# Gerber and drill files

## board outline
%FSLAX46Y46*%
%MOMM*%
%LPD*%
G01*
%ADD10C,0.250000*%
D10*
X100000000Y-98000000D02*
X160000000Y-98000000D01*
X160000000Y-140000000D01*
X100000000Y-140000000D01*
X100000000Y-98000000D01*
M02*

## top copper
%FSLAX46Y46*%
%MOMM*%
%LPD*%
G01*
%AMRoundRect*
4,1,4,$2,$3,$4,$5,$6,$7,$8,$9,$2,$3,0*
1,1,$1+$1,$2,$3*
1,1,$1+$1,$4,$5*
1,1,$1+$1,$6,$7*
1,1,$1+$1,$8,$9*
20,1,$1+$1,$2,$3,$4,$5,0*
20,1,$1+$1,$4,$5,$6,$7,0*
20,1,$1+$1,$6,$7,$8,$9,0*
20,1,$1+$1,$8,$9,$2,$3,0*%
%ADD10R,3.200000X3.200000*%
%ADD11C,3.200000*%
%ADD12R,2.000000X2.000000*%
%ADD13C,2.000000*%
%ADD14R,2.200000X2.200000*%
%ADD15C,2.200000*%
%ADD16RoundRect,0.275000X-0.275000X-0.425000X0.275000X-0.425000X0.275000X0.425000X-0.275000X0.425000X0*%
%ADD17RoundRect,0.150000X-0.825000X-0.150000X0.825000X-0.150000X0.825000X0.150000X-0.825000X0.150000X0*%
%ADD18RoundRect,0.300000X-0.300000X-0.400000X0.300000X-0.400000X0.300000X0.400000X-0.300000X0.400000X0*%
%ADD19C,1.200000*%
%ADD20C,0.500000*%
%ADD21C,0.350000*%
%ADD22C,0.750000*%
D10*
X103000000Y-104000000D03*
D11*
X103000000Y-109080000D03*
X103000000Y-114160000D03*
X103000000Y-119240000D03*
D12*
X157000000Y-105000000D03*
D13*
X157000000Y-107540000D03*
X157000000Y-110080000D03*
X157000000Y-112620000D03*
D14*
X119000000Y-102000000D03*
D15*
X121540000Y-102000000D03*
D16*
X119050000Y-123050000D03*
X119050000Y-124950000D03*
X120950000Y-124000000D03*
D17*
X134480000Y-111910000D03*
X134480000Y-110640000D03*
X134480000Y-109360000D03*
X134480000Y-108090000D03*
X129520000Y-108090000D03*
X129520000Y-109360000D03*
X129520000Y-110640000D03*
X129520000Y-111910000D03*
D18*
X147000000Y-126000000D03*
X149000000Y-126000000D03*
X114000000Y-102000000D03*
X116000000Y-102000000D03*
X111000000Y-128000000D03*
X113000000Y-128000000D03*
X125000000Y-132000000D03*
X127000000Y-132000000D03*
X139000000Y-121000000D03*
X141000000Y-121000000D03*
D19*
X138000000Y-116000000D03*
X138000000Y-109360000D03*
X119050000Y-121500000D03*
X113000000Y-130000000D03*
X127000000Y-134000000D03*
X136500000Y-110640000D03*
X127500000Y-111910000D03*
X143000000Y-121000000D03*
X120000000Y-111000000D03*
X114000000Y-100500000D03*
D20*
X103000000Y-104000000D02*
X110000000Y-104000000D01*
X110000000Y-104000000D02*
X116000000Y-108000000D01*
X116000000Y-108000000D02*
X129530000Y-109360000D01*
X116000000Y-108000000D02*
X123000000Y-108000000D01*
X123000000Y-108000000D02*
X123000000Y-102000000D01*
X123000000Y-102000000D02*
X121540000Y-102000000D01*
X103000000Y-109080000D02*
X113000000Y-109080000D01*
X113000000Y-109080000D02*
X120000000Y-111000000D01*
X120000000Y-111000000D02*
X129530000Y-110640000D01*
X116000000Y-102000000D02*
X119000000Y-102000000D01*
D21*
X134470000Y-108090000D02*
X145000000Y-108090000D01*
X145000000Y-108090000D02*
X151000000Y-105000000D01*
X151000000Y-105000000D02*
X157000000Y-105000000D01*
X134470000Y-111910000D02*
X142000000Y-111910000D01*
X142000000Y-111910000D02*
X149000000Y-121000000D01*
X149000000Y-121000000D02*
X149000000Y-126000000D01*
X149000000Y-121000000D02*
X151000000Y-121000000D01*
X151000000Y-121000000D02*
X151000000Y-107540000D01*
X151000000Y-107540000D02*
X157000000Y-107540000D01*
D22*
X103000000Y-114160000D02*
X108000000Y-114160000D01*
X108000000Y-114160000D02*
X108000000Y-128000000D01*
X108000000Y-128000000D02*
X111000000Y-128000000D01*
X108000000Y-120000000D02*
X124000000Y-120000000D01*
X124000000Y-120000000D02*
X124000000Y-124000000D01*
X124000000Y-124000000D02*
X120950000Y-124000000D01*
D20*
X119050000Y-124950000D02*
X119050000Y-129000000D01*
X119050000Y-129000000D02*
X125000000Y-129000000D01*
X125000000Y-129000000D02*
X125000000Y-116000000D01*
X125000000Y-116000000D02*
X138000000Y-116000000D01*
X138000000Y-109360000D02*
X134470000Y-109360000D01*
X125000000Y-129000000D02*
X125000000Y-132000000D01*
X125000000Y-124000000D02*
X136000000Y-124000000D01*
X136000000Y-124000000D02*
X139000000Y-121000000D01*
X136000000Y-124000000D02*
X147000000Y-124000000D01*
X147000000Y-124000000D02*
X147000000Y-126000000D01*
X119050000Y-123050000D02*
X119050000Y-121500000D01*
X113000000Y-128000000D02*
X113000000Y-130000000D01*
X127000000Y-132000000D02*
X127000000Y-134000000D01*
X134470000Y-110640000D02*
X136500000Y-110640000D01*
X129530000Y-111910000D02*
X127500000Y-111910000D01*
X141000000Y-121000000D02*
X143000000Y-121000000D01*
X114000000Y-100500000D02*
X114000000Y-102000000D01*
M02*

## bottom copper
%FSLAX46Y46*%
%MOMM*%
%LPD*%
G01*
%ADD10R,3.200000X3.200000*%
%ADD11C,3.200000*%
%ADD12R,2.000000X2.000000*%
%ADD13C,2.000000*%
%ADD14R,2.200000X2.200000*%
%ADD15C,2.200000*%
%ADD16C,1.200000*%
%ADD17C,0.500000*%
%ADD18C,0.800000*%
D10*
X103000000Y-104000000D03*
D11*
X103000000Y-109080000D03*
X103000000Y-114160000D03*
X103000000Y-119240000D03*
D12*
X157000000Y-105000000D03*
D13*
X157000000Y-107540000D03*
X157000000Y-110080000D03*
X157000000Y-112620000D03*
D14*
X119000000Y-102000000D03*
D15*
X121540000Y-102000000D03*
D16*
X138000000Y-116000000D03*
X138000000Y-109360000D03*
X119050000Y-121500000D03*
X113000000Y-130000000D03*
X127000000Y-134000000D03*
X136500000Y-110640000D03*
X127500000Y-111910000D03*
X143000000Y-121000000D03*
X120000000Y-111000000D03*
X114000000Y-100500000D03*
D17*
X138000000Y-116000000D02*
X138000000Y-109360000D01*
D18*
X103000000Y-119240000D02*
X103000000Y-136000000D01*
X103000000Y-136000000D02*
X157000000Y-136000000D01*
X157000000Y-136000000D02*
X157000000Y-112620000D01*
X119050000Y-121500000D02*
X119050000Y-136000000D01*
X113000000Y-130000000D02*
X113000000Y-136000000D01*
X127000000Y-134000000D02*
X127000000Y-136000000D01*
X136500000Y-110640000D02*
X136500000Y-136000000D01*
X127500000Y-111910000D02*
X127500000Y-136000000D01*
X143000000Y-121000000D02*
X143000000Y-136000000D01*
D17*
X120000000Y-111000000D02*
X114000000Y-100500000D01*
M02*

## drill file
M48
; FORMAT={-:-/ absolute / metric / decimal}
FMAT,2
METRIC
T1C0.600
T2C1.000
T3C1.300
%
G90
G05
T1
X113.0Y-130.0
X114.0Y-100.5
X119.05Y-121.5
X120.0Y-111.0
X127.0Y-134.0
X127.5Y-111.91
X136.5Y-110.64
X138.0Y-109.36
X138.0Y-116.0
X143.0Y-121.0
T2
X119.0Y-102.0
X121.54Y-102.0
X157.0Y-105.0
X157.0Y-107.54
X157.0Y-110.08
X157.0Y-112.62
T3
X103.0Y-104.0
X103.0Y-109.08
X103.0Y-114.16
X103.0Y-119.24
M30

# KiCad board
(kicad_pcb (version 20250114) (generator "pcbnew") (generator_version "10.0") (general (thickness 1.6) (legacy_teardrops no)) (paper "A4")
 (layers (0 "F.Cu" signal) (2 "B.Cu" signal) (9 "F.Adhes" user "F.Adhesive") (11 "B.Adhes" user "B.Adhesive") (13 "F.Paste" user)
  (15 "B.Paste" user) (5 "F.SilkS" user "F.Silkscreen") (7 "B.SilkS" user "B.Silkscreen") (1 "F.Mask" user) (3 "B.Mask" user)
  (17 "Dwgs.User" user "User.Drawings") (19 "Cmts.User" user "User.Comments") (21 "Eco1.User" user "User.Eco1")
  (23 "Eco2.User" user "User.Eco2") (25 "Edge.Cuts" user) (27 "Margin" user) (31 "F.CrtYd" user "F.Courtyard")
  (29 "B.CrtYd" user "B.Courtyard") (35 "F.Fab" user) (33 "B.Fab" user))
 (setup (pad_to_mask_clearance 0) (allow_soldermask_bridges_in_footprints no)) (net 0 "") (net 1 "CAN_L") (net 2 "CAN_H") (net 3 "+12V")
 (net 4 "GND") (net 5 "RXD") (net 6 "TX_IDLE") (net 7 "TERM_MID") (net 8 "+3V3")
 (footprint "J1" (layer "F.Cu") (at 103.00 104.00 0)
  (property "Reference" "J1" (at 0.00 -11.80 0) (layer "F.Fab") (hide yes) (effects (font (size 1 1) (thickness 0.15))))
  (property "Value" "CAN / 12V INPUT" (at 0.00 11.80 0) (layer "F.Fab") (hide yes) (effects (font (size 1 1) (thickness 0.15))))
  (pad "1" thru_hole rect (at 0.00 0.00) (size 3.20 3.20) (drill 1.30) (layers "*.Cu" "*.Mask") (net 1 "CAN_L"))
  (pad "2" thru_hole circle (at 0.00 5.08) (size 3.20 3.20) (drill 1.30) (layers "*.Cu" "*.Mask") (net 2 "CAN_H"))
  (pad "3" thru_hole circle (at 0.00 10.16) (size 3.20 3.20) (drill 1.30) (layers "*.Cu" "*.Mask") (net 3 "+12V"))
  (pad "4" thru_hole circle (at 0.00 15.24) (size 3.20 3.20) (drill 1.30) (layers "*.Cu" "*.Mask") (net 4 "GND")))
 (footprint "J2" (layer "F.Cu") (at 157.00 105.00 0)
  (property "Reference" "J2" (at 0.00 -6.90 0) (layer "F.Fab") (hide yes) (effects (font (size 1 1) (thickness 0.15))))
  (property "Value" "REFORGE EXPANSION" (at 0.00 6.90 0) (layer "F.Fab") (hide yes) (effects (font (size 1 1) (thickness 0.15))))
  (pad "1" thru_hole rect (at 0.00 0.00) (size 2.00 2.00) (drill 1.00) (layers "*.Cu" "*.Mask") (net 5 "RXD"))
  (pad "2" thru_hole circle (at 0.00 2.54) (size 2.00 2.00) (drill 1.00) (layers "*.Cu" "*.Mask") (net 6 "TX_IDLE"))
  (pad "3" thru_hole circle (at 0.00 5.08) (size 2.00 2.00) (drill 1.00) (layers "*.Cu" "*.Mask") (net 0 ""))
  (pad "4" thru_hole circle (at 0.00 7.62) (size 2.00 2.00) (drill 1.00) (layers "*.Cu" "*.Mask") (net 4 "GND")))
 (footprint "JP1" (layer "F.Cu") (at 119.00 102.00 0)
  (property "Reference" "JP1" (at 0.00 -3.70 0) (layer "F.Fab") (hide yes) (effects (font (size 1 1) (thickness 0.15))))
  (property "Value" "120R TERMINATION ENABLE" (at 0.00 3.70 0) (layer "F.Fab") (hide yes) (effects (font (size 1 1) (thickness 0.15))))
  (pad "1" thru_hole rect (at 0.00 0.00) (size 2.20 2.20) (drill 1.00) (layers "*.Cu" "*.Mask") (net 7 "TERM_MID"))
  (pad "2" thru_hole circle (at 2.54 0.00) (size 2.20 2.20) (drill 1.00) (layers "*.Cu" "*.Mask") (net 1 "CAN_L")))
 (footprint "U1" (layer "F.Cu") (at 120.00 124.00 0)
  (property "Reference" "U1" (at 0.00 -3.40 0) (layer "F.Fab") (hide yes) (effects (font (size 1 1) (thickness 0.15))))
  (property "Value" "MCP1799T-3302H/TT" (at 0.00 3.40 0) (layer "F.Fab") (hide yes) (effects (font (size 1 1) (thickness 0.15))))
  (pad "1" smd roundrect (at -0.95 -0.95) (size 1.10 1.40) (layers "F.Cu" "F.Paste" "F.Mask") (roundrect_rratio 0.25) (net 4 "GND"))
  (pad "2" smd roundrect (at -0.95 0.95) (size 1.10 1.40) (layers "F.Cu" "F.Paste" "F.Mask") (roundrect_rratio 0.25) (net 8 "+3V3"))
  (pad "3" smd roundrect (at 0.95 0.00) (size 1.10 1.40) (layers "F.Cu" "F.Paste" "F.Mask") (roundrect_rratio 0.25) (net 3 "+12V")))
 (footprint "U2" (layer "F.Cu") (at 132.00 110.00 180)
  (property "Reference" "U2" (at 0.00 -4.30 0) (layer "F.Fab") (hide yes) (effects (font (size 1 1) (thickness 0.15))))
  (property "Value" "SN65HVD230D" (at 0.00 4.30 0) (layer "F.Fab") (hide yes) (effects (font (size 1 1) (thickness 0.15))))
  (pad "1" smd roundrect (at -2.48 -1.91) (size 1.95 0.60) (layers "F.Cu" "F.Paste" "F.Mask") (roundrect_rratio 0.25) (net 6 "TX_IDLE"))
  (pad "2" smd roundrect (at -2.48 -0.64) (size 1.95 0.60) (layers "F.Cu" "F.Paste" "F.Mask") (roundrect_rratio 0.25) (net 4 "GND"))
  (pad "3" smd roundrect (at -2.48 0.64) (size 1.95 0.60) (layers "F.Cu" "F.Paste" "F.Mask") (roundrect_rratio 0.25) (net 8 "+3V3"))
  (pad "4" smd roundrect (at -2.48 1.91) (size 1.95 0.60) (layers "F.Cu" "F.Paste" "F.Mask") (roundrect_rratio 0.25) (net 5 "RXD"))
  (pad "5" smd roundrect (at 2.48 1.91) (size 1.95 0.60) (layers "F.Cu" "F.Paste" "F.Mask") (roundrect_rratio 0.25) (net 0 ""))
  (pad "6" smd roundrect (at 2.48 0.64) (size 1.95 0.60) (layers "F.Cu" "F.Paste" "F.Mask") (roundrect_rratio 0.25) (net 1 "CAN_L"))
  (pad "7" smd roundrect (at 2.48 -0.64) (size 1.95 0.60) (layers "F.Cu" "F.Paste" "F.Mask") (roundrect_rratio 0.25) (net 2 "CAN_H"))
  (pad "8" smd roundrect (at 2.48 -1.91) (size 1.95 0.60) (layers "F.Cu" "F.Paste" "F.Mask") (roundrect_rratio 0.25) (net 4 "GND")))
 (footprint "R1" (layer "F.Cu") (at 148.00 126.00 0)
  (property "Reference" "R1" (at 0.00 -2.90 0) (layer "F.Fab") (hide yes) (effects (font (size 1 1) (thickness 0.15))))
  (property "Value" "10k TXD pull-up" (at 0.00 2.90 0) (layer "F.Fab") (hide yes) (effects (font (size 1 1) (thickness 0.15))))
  (pad "1" smd roundrect (at -1.00 0.00) (size 1.20 1.40) (layers "F.Cu" "F.Paste" "F.Mask") (roundrect_rratio 0.25) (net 8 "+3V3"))
  (pad "2" smd roundrect (at 1.00 0.00) (size 1.20 1.40) (layers "F.Cu" "F.Paste" "F.Mask") (roundrect_rratio 0.25) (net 6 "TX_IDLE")))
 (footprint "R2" (layer "F.Cu") (at 115.00 102.00 0)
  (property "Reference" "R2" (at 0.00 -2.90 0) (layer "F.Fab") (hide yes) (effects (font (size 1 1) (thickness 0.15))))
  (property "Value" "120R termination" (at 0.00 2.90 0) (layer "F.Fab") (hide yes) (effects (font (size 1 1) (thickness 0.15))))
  (pad "1" smd roundrect (at -1.00 0.00) (size 1.20 1.40) (layers "F.Cu" "F.Paste" "F.Mask") (roundrect_rratio 0.25) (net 2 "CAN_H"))
  (pad "2" smd roundrect (at 1.00 0.00) (size 1.20 1.40) (layers "F.Cu" "F.Paste" "F.Mask") (roundrect_rratio 0.25) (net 7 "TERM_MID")))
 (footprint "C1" (layer "F.Cu") (at 112.00 128.00 0)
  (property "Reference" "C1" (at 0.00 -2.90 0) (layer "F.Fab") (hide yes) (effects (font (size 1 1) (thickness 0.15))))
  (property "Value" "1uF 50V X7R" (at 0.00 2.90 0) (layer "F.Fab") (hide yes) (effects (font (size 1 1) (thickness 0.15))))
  (pad "1" smd roundrect (at -1.00 0.00) (size 1.20 1.40) (layers "F.Cu" "F.Paste" "F.Mask") (roundrect_rratio 0.25) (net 3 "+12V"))
  (pad "2" smd roundrect (at 1.00 0.00) (size 1.20 1.40) (layers "F.Cu" "F.Paste" "F.Mask") (roundrect_rratio 0.25) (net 4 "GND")))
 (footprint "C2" (layer "F.Cu") (at 126.00 132.00 0)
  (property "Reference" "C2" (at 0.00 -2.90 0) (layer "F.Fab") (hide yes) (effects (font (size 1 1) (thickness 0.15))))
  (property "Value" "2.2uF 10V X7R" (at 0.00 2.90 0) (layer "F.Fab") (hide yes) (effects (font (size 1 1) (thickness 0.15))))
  (pad "1" smd roundrect (at -1.00 0.00) (size 1.20 1.40) (layers "F.Cu" "F.Paste" "F.Mask") (roundrect_rratio 0.25) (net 8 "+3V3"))
  (pad "2" smd roundrect (at 1.00 0.00) (size 1.20 1.40) (layers "F.Cu" "F.Paste" "F.Mask") (roundrect_rratio 0.25) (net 4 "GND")))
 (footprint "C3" (layer "F.Cu") (at 140.00 121.00 0)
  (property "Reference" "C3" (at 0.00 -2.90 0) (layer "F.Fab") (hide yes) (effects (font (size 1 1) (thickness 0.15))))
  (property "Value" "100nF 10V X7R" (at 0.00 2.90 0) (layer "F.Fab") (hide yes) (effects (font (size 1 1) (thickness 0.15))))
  (pad "1" smd roundrect (at -1.00 0.00) (size 1.20 1.40) (layers "F.Cu" "F.Paste" "F.Mask") (roundrect_rratio 0.25) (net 8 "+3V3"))
  (pad "2" smd roundrect (at 1.00 0.00) (size 1.20 1.40) (layers "F.Cu" "F.Paste" "F.Mask") (roundrect_rratio 0.25) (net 4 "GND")))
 (gr_rect (start 100 98) (end 160 140) (stroke (width 0.25) (type default)) (fill none) (layer "Edge.Cuts"))
 (segment (start 103.00 104.00) (end 110.00 104.00) (width 0.50) (layer "F.Cu") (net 1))
 (segment (start 110.00 104.00) (end 116.00 108.00) (width 0.50) (layer "F.Cu") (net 1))
 (segment (start 116.00 108.00) (end 129.53 109.36) (width 0.50) (layer "F.Cu") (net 1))
 (segment (start 116.00 108.00) (end 123.00 108.00) (width 0.50) (layer "F.Cu") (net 1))
 (segment (start 123.00 108.00) (end 123.00 102.00) (width 0.50) (layer "F.Cu") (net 1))
 (segment (start 123.00 102.00) (end 121.54 102.00) (width 0.50) (layer "F.Cu") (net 1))
 (segment (start 103.00 109.08) (end 113.00 109.08) (width 0.50) (layer "F.Cu") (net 2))
 (segment (start 113.00 109.08) (end 120.00 111.00) (width 0.50) (layer "F.Cu") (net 2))
 (segment (start 120.00 111.00) (end 129.53 110.64) (width 0.50) (layer "F.Cu") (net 2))
 (segment (start 116.00 102.00) (end 119.00 102.00) (width 0.50) (layer "F.Cu") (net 7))
 (segment (start 134.47 108.09) (end 145.00 108.09) (width 0.35) (layer "F.Cu") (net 5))
 (segment (start 145.00 108.09) (end 151.00 105.00) (width 0.35) (layer "F.Cu") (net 5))
 (segment (start 151.00 105.00) (end 157.00 105.00) (width 0.35) (layer "F.Cu") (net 5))
 (segment (start 134.47 111.91) (end 142.00 111.91) (width 0.35) (layer "F.Cu") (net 6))
 (segment (start 142.00 111.91) (end 149.00 121.00) (width 0.35) (layer "F.Cu") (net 6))
 (segment (start 149.00 121.00) (end 149.00 126.00) (width 0.35) (layer "F.Cu") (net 6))
 (segment (start 149.00 121.00) (end 151.00 121.00) (width 0.35) (layer "F.Cu") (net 6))
 (segment (start 151.00 121.00) (end 151.00 107.54) (width 0.35) (layer "F.Cu") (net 6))
 (segment (start 151.00 107.54) (end 157.00 107.54) (width 0.35) (layer "F.Cu") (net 6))
 (segment (start 103.00 114.16) (end 108.00 114.16) (width 0.75) (layer "F.Cu") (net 3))
 (segment (start 108.00 114.16) (end 108.00 128.00) (width 0.75) (layer "F.Cu") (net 3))
 (segment (start 108.00 128.00) (end 111.00 128.00) (width 0.75) (layer "F.Cu") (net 3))
 (segment (start 108.00 120.00) (end 124.00 120.00) (width 0.75) (layer "F.Cu") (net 3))
 (segment (start 124.00 120.00) (end 124.00 124.00) (width 0.75) (layer "F.Cu") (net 3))
 (segment (start 124.00 124.00) (end 120.95 124.00) (width 0.75) (layer "F.Cu") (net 3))
 (segment (start 119.05 124.95) (end 119.05 129.00) (width 0.50) (layer "F.Cu") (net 8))
 (segment (start 119.05 129.00) (end 125.00 129.00) (width 0.50) (layer "F.Cu") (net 8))
 (segment (start 125.00 129.00) (end 125.00 116.00) (width 0.50) (layer "F.Cu") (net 8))
 (segment (start 125.00 116.00) (end 138.00 116.00) (width 0.50) (layer "F.Cu") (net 8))
 (segment (start 138.00 109.36) (end 134.47 109.36) (width 0.50) (layer "F.Cu") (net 8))
 (segment (start 125.00 129.00) (end 125.00 132.00) (width 0.50) (layer "F.Cu") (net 8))
 (segment (start 125.00 124.00) (end 136.00 124.00) (width 0.50) (layer "F.Cu") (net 8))
 (segment (start 136.00 124.00) (end 139.00 121.00) (width 0.50) (layer "F.Cu") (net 8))
 (segment (start 136.00 124.00) (end 147.00 124.00) (width 0.50) (layer "F.Cu") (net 8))
 (segment (start 147.00 124.00) (end 147.00 126.00) (width 0.50) (layer "F.Cu") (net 8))
 (segment (start 138.00 116.00) (end 138.00 109.36) (width 0.50) (layer "B.Cu") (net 8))
 (segment (start 119.05 123.05) (end 119.05 121.50) (width 0.50) (layer "F.Cu") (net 4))
 (segment (start 113.00 128.00) (end 113.00 130.00) (width 0.50) (layer "F.Cu") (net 4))
 (segment (start 127.00 132.00) (end 127.00 134.00) (width 0.50) (layer "F.Cu") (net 4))
 (segment (start 134.47 110.64) (end 136.50 110.64) (width 0.50) (layer "F.Cu") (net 4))
 (segment (start 129.53 111.91) (end 127.50 111.91) (width 0.50) (layer "F.Cu") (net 4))
 (segment (start 141.00 121.00) (end 143.00 121.00) (width 0.50) (layer "F.Cu") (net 4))
 (segment (start 103.00 119.24) (end 103.00 136.00) (width 0.80) (layer "B.Cu") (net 4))
 (segment (start 103.00 136.00) (end 157.00 136.00) (width 0.80) (layer "B.Cu") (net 4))
 (segment (start 157.00 136.00) (end 157.00 112.62) (width 0.80) (layer "B.Cu") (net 4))
 (segment (start 119.05 121.50) (end 119.05 136.00) (width 0.80) (layer "B.Cu") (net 4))
 (segment (start 113.00 130.00) (end 113.00 136.00) (width 0.80) (layer "B.Cu") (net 4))
 (segment (start 127.00 134.00) (end 127.00 136.00) (width 0.80) (layer "B.Cu") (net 4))
 (segment (start 136.50 110.64) (end 136.50 136.00) (width 0.80) (layer "B.Cu") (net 4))
 (segment (start 127.50 111.91) (end 127.50 136.00) (width 0.80) (layer "B.Cu") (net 4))
 (segment (start 143.00 121.00) (end 143.00 136.00) (width 0.80) (layer "B.Cu") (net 4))
 (segment (start 120.00 111.00) (end 114.00 100.50) (width 0.50) (layer "B.Cu") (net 2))
 (segment (start 114.00 100.50) (end 114.00 102.00) (width 0.50) (layer "F.Cu") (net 2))
 (via (at 138.00 116.00) (size 1.2) (drill 0.6) (layers "F.Cu" "B.Cu") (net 8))
 (via (at 138.00 109.36) (size 1.2) (drill 0.6) (layers "F.Cu" "B.Cu") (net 8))
 (via (at 119.05 121.50) (size 1.2) (drill 0.6) (layers "F.Cu" "B.Cu") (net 4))
 (via (at 113.00 130.00) (size 1.2) (drill 0.6) (layers "F.Cu" "B.Cu") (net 4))
 (via (at 127.00 134.00) (size 1.2) (drill 0.6) (layers "F.Cu" "B.Cu") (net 4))
 (via (at 136.50 110.64) (size 1.2) (drill 0.6) (layers "F.Cu" "B.Cu") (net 4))
 (via (at 127.50 111.91) (size 1.2) (drill 0.6) (layers "F.Cu" "B.Cu") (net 4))
 (via (at 143.00 121.00) (size 1.2) (drill 0.6) (layers "F.Cu" "B.Cu") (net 4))
 (via (at 120.00 111.00) (size 1.2) (drill 0.6) (layers "F.Cu" "B.Cu") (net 2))
 (via (at 114.00 100.50) (size 1.2) (drill 0.6) (layers "F.Cu" "B.Cu") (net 2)))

